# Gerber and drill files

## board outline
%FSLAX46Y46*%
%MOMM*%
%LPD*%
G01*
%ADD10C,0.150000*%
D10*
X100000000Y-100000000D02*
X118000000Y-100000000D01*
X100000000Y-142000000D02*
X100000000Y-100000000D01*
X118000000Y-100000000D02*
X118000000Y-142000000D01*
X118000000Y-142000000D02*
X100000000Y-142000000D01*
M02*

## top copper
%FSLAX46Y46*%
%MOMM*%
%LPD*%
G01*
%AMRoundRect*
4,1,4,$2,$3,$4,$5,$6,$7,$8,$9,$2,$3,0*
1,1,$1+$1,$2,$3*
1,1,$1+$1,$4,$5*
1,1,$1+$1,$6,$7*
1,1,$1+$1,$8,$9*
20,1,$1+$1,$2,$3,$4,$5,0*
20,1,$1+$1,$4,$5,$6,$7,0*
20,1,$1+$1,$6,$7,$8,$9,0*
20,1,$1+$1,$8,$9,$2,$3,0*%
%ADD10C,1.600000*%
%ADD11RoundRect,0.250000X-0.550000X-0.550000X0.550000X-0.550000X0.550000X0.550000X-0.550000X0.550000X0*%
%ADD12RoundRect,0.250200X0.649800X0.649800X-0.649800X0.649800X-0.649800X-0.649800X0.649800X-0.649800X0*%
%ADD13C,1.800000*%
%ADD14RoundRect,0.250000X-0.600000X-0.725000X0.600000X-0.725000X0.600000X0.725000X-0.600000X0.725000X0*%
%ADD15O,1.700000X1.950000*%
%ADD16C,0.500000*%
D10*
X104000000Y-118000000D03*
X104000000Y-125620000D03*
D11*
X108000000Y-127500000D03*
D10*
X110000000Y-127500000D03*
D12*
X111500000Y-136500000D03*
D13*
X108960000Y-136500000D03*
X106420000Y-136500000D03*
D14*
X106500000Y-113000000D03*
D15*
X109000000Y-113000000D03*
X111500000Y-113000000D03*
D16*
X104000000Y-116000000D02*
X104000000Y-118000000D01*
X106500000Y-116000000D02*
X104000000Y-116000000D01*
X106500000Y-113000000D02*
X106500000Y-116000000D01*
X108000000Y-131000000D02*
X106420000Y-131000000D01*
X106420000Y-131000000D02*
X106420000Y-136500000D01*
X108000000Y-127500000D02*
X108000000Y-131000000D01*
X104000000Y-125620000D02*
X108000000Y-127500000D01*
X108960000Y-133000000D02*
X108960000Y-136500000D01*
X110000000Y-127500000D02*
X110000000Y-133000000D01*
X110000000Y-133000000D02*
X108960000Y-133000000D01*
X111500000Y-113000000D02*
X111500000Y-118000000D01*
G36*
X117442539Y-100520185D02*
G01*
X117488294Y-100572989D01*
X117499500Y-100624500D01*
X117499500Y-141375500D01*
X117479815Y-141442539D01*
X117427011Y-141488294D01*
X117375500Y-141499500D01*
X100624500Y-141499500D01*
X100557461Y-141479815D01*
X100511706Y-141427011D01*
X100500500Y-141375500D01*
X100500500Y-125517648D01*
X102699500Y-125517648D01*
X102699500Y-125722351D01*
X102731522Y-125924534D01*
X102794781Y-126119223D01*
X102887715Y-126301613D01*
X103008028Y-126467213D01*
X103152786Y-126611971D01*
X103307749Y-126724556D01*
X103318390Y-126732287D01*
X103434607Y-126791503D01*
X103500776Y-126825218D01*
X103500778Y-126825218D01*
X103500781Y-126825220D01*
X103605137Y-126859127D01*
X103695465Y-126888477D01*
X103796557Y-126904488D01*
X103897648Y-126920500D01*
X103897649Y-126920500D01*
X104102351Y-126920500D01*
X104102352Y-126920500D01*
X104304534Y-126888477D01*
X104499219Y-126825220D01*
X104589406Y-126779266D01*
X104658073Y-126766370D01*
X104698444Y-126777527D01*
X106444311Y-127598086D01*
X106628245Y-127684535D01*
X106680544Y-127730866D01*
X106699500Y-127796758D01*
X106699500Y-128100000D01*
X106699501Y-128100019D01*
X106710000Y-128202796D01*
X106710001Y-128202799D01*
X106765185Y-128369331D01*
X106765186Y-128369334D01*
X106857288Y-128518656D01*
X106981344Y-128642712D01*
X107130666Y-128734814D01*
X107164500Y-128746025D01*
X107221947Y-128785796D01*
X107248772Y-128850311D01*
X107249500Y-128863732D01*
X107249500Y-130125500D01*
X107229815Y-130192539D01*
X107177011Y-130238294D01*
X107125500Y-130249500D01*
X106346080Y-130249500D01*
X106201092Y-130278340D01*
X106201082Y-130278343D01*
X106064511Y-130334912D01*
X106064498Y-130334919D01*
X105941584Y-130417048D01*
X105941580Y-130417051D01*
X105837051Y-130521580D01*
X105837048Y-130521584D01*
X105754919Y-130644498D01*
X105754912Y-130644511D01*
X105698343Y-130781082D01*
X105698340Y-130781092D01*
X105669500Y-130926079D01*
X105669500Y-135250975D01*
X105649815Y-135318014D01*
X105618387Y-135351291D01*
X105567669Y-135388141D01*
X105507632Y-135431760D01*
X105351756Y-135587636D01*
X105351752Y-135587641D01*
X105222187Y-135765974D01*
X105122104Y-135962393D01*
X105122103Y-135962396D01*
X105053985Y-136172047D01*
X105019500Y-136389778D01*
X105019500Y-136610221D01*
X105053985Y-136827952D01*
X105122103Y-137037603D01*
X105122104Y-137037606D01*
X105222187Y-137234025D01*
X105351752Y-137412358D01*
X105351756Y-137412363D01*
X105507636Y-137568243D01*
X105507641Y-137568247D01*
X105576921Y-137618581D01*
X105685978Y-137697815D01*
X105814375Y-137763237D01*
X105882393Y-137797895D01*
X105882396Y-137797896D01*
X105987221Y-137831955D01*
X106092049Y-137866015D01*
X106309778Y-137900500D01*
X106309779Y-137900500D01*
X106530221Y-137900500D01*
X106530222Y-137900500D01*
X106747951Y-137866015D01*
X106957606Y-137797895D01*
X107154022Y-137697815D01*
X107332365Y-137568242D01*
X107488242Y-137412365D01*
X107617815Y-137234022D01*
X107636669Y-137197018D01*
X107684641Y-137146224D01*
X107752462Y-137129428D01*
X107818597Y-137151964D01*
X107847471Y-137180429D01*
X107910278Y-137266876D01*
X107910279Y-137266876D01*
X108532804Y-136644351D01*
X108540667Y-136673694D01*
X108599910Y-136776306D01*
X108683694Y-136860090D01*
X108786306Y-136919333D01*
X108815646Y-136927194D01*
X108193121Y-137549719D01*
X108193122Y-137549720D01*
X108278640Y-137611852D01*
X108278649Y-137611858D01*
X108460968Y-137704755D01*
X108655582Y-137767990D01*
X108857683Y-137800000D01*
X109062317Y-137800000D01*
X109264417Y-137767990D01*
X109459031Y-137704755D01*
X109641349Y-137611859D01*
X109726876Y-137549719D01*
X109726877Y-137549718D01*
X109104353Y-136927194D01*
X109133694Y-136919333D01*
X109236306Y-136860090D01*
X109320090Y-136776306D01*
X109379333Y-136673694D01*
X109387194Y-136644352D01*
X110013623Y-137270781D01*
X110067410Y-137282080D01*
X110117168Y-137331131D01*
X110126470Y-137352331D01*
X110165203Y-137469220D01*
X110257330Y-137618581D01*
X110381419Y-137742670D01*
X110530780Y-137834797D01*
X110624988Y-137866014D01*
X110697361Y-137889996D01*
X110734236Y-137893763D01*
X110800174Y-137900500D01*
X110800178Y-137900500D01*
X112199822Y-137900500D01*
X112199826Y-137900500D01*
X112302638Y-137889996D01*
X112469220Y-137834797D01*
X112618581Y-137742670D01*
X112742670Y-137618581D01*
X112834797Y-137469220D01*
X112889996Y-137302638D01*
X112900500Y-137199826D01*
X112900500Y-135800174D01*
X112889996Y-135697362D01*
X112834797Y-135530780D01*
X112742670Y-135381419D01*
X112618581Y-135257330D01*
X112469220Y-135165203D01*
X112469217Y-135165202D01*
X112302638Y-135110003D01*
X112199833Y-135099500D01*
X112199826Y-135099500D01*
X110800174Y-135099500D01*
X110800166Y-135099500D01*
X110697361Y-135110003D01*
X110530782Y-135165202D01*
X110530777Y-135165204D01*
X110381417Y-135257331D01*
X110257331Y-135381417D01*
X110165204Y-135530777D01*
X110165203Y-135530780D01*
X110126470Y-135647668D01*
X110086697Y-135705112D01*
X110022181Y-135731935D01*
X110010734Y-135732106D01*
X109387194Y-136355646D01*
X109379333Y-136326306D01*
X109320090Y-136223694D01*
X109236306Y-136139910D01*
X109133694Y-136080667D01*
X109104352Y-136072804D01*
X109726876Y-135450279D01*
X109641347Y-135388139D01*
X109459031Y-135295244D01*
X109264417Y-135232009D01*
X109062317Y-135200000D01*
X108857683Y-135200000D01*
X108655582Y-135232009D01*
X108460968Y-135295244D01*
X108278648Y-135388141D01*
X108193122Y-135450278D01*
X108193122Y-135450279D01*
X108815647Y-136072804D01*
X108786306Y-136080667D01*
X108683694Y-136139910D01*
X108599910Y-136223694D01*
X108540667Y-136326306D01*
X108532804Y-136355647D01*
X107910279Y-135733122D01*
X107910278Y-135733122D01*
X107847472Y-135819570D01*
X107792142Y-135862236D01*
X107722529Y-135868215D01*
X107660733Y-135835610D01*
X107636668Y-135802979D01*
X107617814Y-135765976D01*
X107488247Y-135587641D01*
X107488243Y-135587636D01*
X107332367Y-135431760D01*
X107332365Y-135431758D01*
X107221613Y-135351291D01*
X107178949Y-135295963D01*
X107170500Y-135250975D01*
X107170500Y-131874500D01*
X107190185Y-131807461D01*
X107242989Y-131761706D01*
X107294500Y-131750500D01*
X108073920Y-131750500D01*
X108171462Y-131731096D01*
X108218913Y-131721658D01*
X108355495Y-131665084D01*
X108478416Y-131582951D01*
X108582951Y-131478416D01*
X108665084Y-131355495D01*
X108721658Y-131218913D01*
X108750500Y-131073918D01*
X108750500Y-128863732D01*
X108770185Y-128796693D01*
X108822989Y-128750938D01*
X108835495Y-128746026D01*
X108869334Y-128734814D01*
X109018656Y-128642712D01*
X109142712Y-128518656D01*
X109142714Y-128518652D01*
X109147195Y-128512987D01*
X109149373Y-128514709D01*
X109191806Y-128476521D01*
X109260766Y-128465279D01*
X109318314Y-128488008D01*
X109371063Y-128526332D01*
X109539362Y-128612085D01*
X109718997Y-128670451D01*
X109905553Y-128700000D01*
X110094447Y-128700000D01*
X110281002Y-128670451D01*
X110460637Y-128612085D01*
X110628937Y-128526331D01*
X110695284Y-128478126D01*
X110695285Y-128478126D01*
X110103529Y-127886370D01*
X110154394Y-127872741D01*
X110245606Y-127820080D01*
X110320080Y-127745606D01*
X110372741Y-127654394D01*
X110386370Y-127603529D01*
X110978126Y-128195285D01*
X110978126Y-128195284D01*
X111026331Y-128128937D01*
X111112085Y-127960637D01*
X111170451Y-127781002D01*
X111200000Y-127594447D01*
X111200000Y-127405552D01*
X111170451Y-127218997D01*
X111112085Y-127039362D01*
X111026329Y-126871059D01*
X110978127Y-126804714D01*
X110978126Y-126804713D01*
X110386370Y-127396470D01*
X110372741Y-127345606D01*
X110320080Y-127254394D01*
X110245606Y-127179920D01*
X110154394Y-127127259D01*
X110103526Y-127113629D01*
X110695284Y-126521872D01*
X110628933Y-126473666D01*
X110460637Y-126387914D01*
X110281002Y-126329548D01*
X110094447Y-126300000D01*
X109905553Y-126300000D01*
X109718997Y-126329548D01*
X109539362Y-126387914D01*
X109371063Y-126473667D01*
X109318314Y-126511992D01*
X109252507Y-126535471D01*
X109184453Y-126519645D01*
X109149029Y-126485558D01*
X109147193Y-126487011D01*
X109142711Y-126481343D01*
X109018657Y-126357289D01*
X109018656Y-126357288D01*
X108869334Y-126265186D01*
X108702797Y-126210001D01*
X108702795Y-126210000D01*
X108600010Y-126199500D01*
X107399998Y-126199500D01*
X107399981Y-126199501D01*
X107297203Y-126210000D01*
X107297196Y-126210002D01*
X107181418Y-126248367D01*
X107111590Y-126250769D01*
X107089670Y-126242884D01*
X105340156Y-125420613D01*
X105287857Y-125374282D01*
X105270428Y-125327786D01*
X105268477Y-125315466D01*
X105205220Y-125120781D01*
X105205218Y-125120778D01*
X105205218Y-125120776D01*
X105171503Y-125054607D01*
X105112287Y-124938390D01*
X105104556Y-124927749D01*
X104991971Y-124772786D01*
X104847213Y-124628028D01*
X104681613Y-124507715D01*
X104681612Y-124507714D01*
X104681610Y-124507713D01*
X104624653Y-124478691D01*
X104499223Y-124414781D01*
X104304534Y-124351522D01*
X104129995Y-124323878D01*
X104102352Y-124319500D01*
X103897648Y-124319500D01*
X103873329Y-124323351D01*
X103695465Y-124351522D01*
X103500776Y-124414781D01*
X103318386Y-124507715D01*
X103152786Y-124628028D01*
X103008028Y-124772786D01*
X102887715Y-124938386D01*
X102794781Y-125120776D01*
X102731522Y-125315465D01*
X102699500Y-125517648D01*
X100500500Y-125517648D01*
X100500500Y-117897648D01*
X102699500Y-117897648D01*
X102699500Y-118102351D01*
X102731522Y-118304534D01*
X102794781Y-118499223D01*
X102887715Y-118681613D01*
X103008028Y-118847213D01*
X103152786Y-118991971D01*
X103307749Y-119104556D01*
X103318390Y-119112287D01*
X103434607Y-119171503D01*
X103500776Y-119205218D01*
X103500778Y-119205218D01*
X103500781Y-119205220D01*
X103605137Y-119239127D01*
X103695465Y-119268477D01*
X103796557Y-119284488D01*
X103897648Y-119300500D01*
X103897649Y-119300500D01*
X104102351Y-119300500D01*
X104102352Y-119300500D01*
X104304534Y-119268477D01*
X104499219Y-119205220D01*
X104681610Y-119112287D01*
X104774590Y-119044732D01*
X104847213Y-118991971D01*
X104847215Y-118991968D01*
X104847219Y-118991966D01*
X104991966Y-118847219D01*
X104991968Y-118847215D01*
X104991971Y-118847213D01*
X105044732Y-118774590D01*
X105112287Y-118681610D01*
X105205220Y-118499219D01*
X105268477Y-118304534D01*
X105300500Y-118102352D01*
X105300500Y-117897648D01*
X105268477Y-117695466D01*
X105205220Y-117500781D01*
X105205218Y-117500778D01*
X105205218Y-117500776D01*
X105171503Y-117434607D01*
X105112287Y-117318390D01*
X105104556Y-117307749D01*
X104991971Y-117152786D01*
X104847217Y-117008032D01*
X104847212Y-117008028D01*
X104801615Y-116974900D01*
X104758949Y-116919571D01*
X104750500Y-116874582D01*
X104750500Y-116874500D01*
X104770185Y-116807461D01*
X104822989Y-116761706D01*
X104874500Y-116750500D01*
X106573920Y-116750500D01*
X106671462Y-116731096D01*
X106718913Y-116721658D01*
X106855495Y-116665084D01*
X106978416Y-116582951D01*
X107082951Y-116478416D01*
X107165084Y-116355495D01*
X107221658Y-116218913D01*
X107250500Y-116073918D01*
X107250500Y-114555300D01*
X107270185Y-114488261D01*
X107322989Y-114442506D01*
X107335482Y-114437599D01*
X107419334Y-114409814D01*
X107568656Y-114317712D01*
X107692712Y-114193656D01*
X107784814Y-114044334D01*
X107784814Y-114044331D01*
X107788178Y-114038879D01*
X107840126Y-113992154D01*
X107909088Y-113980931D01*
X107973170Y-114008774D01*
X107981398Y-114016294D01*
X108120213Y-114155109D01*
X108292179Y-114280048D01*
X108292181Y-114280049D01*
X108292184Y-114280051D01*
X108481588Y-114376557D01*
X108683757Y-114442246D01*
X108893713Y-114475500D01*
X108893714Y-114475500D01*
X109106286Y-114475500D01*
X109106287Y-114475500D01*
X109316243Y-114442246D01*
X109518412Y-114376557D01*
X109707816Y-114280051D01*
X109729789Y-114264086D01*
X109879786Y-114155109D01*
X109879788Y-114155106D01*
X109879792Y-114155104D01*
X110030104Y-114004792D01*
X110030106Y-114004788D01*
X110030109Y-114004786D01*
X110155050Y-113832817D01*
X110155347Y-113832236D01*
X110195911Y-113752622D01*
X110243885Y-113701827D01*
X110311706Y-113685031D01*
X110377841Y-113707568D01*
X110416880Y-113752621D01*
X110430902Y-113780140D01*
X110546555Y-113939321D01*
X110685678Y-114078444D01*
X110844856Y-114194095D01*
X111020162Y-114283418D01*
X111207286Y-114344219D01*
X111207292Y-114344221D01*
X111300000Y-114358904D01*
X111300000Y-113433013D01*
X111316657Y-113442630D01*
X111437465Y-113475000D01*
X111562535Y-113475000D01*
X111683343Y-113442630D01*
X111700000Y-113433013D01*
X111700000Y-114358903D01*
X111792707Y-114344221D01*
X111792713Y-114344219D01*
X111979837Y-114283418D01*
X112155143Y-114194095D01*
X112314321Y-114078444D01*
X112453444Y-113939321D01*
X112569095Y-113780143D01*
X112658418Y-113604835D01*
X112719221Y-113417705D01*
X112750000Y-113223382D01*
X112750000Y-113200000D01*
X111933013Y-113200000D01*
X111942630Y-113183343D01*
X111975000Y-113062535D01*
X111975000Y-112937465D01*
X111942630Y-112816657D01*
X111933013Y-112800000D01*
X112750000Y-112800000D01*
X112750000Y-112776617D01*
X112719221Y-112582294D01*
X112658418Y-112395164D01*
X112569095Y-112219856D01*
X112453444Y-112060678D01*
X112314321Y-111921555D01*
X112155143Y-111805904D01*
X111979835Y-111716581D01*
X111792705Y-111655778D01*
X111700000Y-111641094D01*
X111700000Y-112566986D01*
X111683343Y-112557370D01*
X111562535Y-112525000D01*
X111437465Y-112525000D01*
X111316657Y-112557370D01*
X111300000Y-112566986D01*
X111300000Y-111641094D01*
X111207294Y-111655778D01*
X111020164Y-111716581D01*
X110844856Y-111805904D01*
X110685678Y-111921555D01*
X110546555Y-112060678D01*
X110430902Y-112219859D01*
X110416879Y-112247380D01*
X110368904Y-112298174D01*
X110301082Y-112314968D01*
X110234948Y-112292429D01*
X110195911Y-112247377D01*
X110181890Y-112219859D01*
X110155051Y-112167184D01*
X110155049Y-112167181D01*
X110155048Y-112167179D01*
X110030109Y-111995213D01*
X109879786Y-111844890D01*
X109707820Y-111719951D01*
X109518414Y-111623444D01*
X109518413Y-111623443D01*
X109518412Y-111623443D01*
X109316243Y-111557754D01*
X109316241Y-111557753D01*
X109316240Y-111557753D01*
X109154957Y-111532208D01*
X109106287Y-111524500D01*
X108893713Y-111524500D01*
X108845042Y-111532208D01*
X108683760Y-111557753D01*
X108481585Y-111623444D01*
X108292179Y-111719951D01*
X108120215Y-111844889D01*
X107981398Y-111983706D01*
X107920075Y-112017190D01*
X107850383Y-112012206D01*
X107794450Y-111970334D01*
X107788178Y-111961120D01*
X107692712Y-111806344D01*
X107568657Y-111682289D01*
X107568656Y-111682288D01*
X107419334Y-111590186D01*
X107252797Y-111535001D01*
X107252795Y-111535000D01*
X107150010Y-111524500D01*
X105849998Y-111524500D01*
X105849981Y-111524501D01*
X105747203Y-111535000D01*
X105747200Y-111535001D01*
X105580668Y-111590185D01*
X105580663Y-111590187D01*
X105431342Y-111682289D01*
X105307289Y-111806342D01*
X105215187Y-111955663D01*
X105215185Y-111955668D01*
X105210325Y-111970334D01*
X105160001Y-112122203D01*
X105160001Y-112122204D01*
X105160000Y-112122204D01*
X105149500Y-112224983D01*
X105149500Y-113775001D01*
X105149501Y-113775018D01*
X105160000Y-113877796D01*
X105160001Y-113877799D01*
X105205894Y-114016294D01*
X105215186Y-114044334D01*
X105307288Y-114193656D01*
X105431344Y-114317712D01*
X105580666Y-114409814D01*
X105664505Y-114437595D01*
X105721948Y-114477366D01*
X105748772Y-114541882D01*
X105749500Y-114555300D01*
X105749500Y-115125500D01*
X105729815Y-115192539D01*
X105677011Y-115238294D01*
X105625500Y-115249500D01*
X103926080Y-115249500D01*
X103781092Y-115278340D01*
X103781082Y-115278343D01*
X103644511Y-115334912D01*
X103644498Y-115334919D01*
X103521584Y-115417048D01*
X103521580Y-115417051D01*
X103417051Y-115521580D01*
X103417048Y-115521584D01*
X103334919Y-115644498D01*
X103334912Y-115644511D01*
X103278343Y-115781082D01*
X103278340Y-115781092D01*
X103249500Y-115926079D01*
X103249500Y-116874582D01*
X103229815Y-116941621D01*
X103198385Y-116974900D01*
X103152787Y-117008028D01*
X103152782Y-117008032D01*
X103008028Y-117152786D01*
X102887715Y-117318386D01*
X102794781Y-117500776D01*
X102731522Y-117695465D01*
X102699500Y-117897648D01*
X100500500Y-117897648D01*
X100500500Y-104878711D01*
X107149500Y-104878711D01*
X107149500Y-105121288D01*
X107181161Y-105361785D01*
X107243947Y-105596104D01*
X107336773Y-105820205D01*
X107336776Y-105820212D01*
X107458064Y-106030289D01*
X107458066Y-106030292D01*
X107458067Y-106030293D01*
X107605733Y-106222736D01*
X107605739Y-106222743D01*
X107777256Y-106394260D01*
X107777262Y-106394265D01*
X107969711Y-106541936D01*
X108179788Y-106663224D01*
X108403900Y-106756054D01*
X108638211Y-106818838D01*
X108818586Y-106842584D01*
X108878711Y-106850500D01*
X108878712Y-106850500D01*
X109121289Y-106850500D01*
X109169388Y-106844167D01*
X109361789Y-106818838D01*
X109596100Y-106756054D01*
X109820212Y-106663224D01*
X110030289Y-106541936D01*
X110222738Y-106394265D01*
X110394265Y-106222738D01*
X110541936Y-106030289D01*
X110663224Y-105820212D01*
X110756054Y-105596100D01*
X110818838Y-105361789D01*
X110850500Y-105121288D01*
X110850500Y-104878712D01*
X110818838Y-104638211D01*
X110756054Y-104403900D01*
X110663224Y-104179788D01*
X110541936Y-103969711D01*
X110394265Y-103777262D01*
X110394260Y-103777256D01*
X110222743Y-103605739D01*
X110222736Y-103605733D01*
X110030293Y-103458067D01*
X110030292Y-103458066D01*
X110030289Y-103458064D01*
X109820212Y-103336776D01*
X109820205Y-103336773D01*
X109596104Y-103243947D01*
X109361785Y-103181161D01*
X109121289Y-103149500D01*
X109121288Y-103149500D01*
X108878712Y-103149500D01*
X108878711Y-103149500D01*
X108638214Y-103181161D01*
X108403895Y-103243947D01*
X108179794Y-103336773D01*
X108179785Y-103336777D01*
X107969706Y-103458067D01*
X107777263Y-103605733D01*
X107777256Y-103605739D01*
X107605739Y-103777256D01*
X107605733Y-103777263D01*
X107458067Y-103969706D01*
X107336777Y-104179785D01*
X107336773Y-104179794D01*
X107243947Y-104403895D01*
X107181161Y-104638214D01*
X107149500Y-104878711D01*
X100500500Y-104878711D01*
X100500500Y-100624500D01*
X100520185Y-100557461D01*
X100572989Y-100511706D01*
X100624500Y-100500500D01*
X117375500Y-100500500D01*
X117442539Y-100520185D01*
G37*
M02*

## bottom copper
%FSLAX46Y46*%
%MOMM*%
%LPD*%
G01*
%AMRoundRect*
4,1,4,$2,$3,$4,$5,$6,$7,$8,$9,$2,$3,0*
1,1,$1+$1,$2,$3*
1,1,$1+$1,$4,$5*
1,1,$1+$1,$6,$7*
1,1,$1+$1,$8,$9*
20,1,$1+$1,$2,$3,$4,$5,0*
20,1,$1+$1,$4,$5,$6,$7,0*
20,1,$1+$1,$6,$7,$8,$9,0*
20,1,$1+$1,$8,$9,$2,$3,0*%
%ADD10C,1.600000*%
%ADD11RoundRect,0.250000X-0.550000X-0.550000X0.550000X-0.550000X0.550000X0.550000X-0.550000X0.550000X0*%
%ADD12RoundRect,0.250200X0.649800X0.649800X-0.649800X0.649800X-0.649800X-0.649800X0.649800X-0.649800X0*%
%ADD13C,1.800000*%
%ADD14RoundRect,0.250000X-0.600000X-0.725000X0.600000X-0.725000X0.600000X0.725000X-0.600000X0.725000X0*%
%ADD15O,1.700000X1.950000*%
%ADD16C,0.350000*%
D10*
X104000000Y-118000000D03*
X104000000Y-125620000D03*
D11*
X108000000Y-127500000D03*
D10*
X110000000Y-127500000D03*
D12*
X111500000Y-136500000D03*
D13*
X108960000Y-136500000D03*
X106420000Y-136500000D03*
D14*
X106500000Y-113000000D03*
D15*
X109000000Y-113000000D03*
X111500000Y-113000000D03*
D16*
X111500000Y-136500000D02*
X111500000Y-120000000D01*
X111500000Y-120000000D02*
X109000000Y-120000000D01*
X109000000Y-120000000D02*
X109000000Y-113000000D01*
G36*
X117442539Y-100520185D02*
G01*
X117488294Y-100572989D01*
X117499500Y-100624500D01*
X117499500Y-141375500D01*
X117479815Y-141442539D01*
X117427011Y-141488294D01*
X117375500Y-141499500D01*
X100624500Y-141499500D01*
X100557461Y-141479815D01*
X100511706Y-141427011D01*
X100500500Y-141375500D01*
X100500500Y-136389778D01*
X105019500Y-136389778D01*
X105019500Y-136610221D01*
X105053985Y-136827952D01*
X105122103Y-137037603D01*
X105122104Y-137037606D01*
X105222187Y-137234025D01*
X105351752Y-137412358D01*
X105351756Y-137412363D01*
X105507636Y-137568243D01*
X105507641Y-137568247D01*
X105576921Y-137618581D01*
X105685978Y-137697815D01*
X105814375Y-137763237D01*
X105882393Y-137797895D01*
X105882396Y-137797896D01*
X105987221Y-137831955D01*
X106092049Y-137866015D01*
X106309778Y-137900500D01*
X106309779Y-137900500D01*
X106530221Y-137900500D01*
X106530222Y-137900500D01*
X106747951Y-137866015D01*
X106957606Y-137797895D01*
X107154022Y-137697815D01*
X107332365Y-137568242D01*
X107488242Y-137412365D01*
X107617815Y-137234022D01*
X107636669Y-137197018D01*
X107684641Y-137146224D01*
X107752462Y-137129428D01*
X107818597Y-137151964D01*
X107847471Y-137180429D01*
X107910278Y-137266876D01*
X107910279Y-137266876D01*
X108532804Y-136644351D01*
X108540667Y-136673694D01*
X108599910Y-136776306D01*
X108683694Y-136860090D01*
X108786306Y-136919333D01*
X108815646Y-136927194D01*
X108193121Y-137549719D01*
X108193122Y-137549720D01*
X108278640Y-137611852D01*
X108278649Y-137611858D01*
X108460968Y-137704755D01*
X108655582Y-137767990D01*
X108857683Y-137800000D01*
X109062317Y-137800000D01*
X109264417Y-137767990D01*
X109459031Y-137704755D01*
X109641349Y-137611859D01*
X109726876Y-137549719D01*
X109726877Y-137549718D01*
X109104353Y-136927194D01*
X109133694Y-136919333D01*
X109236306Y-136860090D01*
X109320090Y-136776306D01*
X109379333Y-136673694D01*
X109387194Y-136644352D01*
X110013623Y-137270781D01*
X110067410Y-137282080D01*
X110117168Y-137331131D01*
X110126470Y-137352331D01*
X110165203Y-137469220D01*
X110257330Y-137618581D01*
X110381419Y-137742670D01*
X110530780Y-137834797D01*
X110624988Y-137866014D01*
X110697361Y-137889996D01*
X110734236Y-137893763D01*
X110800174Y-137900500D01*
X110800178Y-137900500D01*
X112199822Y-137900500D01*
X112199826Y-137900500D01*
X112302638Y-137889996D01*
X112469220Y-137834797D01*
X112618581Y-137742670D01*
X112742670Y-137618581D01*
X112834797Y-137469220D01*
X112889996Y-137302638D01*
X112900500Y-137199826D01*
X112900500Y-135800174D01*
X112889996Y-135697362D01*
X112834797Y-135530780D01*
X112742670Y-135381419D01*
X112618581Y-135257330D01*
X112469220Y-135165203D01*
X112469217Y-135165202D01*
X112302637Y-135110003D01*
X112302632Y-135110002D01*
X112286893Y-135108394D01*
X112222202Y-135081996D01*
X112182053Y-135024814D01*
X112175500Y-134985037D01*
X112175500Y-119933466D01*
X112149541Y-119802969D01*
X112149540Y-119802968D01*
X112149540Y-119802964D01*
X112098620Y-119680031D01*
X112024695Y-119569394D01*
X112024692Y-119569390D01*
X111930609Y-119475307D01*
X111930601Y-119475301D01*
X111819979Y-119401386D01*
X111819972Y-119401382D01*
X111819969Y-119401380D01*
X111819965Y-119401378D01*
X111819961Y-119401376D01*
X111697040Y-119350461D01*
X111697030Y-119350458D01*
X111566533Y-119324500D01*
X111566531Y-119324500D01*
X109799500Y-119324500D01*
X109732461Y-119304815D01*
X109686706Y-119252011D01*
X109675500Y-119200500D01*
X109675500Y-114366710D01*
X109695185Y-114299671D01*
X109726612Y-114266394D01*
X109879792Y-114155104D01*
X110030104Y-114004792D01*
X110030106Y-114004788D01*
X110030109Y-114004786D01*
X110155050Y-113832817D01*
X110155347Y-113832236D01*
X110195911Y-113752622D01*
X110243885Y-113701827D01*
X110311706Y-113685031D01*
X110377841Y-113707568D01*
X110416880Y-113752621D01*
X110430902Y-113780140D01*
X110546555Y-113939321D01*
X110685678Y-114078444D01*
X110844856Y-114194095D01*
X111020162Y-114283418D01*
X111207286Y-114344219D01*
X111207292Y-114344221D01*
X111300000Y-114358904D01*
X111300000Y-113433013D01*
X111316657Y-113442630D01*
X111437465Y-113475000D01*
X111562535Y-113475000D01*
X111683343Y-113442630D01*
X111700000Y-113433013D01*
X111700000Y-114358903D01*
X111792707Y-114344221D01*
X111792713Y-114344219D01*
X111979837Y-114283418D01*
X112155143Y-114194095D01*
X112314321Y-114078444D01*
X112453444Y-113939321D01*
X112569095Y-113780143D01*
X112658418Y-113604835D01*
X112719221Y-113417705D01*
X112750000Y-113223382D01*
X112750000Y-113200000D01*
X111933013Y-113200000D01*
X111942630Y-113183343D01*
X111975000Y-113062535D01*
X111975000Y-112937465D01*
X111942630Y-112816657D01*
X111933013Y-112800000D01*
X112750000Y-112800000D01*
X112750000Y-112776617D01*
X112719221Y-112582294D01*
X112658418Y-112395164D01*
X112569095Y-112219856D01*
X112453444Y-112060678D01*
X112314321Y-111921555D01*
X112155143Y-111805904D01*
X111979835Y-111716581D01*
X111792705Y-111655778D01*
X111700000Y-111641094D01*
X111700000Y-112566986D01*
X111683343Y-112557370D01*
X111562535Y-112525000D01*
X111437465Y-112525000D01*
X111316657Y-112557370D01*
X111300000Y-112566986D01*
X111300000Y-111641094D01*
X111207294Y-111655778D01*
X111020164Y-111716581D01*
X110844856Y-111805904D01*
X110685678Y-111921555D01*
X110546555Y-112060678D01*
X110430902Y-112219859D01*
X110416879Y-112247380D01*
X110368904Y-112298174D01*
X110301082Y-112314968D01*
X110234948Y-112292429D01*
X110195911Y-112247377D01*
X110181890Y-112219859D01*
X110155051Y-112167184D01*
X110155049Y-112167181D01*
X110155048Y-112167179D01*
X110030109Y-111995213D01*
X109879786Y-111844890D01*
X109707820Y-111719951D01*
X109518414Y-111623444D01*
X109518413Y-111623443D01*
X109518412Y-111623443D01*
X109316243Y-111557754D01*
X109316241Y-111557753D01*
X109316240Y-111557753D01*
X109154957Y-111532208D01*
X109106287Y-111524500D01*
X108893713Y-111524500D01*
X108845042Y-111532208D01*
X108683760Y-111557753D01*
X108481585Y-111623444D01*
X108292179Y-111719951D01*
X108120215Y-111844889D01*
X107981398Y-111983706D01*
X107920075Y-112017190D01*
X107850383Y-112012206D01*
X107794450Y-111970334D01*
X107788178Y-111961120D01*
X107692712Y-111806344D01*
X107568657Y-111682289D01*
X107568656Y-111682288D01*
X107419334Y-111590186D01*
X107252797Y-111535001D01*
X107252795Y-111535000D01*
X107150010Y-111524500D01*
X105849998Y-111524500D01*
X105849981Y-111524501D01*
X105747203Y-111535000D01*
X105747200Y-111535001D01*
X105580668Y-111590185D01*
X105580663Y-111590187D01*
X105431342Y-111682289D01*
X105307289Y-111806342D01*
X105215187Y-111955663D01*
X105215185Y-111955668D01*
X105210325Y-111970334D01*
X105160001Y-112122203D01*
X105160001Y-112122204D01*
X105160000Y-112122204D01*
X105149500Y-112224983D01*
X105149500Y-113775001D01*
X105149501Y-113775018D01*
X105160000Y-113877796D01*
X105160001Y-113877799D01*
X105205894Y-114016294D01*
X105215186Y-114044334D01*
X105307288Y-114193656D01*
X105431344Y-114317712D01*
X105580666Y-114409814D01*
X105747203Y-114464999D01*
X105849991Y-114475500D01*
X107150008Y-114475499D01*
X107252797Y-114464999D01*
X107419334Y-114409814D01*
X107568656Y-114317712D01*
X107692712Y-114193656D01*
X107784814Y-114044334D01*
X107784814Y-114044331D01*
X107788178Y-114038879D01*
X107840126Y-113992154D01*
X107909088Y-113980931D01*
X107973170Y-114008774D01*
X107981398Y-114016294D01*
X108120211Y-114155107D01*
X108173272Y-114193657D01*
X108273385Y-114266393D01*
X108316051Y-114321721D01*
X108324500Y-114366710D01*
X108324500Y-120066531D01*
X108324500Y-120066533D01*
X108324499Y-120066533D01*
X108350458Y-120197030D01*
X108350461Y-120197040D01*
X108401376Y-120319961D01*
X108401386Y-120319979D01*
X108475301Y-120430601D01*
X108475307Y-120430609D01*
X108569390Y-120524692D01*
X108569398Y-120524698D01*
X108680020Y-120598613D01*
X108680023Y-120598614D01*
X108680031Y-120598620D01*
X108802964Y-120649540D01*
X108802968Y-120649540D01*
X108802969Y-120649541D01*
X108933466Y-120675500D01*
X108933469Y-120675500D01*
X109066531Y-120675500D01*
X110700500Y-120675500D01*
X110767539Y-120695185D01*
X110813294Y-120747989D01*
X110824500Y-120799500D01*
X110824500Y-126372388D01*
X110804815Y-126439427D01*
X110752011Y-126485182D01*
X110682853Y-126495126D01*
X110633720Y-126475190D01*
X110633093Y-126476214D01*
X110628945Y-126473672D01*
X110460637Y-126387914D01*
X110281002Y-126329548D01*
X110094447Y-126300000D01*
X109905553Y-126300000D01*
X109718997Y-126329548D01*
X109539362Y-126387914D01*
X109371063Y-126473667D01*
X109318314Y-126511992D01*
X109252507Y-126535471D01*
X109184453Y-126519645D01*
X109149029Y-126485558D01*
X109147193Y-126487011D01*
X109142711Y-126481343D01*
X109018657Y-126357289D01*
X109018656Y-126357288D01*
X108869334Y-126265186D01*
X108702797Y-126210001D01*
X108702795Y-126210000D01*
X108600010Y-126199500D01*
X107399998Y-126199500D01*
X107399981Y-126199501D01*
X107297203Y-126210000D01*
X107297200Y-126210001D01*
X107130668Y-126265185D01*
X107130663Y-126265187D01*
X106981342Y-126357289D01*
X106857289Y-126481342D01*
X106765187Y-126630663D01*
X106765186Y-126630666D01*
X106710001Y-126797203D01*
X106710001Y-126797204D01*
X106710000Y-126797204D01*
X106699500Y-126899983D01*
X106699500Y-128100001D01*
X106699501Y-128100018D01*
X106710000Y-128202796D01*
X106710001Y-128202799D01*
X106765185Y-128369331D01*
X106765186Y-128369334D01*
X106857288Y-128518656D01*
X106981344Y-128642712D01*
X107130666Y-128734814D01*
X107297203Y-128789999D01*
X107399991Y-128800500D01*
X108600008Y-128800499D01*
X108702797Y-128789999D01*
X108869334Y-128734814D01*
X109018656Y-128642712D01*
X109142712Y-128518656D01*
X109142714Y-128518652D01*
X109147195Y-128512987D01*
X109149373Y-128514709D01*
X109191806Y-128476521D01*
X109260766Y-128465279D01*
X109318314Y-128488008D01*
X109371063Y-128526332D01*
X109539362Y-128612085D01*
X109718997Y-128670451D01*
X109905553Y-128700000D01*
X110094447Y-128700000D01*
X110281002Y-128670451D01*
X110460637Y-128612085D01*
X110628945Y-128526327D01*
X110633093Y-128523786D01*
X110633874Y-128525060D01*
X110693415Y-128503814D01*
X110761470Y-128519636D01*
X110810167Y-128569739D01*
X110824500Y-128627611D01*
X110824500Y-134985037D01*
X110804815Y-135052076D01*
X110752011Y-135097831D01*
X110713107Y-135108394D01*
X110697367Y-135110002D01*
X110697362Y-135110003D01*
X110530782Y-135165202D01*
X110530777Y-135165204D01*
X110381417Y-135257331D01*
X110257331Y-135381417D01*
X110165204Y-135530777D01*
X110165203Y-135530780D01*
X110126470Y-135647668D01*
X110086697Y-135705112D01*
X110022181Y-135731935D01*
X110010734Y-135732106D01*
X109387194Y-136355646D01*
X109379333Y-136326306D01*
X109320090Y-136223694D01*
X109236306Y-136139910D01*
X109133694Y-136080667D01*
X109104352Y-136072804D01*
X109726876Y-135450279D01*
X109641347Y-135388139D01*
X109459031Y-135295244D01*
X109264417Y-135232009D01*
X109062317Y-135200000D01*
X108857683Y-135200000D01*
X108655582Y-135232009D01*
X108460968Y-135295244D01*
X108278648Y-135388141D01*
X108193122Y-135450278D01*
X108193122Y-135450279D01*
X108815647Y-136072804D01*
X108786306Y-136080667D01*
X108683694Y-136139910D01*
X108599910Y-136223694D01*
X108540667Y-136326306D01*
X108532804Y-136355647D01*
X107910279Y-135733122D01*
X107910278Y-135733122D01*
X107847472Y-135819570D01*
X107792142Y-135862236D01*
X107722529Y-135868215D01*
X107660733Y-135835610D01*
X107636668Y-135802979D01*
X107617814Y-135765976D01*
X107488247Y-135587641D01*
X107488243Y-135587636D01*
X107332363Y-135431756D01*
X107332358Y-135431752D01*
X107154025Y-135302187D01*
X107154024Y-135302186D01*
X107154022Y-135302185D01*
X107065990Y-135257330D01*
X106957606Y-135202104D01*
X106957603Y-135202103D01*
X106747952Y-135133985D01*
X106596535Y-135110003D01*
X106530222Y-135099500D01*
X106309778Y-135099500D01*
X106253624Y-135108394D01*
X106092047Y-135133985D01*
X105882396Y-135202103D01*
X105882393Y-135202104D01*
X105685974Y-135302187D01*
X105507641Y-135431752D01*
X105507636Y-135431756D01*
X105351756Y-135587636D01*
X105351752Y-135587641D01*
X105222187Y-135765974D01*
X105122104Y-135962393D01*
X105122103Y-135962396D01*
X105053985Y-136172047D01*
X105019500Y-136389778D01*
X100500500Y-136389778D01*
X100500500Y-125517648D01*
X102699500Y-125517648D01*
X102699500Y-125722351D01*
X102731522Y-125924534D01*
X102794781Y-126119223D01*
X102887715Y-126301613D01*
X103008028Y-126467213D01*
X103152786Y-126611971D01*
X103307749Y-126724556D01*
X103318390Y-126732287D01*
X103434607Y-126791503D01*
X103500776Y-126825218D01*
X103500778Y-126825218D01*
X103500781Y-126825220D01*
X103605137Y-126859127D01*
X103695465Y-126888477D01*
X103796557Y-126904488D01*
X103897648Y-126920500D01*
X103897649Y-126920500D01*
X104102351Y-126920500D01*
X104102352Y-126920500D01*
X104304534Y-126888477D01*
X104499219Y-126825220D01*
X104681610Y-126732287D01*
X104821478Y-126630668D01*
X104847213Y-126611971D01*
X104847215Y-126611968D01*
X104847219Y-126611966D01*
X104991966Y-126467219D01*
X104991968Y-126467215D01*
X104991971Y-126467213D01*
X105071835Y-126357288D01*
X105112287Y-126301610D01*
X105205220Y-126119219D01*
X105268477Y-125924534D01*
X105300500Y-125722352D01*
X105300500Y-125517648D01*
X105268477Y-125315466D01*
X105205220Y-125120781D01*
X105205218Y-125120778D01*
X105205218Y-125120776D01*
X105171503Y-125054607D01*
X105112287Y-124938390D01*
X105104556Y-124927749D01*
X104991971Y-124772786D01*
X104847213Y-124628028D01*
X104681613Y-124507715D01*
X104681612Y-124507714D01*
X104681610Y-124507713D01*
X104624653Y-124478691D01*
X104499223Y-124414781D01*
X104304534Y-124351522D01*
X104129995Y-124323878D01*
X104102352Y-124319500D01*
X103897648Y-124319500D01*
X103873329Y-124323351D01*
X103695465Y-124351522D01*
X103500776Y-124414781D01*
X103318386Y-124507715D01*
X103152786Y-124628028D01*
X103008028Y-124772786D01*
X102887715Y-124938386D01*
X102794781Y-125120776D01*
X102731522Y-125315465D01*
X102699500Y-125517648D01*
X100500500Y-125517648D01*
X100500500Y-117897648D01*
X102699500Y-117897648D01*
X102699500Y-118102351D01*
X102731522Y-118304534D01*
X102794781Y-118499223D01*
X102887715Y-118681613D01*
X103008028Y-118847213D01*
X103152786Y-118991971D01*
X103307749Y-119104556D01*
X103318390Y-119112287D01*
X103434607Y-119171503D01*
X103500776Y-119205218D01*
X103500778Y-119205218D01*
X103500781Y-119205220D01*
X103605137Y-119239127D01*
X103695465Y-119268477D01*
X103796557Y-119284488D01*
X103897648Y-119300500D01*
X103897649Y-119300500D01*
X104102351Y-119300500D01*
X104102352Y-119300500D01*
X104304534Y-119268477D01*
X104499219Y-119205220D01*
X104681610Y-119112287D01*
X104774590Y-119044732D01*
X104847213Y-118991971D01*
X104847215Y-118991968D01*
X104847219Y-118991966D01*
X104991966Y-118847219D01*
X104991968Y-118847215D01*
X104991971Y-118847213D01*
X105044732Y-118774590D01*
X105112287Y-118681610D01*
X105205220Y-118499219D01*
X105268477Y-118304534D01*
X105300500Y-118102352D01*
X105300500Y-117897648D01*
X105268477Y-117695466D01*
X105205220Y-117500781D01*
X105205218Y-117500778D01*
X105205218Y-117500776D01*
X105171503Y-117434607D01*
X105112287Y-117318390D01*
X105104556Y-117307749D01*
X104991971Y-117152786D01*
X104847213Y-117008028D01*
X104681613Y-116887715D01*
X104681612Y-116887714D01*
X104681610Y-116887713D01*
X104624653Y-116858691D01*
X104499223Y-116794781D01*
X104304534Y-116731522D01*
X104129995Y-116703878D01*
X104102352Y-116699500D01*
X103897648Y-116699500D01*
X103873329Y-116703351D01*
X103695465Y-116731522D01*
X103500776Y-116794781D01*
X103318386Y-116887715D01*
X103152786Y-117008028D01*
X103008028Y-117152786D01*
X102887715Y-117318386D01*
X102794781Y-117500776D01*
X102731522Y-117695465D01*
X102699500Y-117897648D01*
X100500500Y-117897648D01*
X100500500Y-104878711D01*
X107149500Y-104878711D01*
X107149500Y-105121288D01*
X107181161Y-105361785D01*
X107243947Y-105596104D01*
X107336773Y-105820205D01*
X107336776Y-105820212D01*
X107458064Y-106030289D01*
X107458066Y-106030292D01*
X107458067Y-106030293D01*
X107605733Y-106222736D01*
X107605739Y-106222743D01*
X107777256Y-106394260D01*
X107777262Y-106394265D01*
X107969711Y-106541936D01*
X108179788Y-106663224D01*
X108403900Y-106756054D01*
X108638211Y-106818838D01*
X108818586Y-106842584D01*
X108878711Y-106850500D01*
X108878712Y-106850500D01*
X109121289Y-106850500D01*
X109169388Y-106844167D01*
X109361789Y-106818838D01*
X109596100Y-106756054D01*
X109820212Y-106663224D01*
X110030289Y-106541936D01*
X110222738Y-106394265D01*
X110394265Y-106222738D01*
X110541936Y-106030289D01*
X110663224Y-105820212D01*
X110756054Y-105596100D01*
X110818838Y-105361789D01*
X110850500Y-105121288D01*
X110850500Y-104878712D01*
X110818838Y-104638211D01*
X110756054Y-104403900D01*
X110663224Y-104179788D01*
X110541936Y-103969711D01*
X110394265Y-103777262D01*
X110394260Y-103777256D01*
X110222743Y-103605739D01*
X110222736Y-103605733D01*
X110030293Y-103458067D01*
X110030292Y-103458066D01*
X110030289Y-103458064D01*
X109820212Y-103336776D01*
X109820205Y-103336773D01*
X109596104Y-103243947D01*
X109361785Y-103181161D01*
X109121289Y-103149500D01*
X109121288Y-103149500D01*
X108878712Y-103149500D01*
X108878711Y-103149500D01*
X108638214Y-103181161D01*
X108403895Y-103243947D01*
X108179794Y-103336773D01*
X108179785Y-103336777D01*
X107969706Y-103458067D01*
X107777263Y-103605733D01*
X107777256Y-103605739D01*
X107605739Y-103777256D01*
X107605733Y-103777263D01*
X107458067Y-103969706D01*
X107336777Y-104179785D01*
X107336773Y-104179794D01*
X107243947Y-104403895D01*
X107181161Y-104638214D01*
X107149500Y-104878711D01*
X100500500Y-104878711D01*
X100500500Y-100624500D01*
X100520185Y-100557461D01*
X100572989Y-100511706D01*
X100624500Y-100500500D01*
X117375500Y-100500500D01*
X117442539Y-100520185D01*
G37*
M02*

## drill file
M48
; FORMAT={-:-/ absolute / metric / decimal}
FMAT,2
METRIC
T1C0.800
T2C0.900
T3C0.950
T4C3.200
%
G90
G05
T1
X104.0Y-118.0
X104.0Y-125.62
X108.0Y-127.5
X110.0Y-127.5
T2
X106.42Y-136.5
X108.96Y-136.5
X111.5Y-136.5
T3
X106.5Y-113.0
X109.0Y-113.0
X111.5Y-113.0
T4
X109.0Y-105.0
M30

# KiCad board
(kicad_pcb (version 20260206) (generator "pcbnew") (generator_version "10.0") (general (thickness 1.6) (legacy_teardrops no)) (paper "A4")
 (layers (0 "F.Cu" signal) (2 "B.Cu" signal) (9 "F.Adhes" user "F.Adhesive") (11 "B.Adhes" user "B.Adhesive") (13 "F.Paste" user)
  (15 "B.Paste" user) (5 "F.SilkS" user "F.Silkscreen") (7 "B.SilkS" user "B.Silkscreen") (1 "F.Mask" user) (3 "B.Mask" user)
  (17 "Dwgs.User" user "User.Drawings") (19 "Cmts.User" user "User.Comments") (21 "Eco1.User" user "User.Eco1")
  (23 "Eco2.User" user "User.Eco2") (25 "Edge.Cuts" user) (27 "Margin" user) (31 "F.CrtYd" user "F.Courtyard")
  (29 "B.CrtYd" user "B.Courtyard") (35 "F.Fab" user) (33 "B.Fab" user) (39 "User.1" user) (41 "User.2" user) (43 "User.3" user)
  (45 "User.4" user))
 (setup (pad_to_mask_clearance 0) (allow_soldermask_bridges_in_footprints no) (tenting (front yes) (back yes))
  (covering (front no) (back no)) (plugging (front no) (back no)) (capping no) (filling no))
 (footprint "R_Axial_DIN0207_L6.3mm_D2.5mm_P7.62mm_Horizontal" (layer "F.Cu") (at 104 118 -90)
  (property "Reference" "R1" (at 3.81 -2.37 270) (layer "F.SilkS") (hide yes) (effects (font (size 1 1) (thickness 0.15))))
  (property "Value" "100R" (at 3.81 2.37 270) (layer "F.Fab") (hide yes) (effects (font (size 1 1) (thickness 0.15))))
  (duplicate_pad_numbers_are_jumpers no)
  (pad "1" thru_hole circle (at 0 0 270) (size 1.6 1.6) (drill 0.8) (layers "*.Cu" "*.Mask") (remove_unused_layers no) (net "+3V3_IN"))
  (pad "2" thru_hole circle (at 7.62 0 270) (size 1.6 1.6) (drill 0.8) (layers "*.Cu" "*.Mask") (remove_unused_layers no) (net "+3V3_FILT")))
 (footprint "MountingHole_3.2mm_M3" (layer "F.Cu") (at 109 105)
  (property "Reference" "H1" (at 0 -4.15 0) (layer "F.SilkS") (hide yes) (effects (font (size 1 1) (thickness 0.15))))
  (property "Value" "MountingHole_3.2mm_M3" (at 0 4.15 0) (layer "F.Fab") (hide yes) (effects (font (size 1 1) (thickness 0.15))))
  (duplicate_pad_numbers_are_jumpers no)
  (pad "" np_thru_hole circle (at 0 0) (size 3.2 3.2) (drill 3.2) (layers "*.Cu" "*.Mask")))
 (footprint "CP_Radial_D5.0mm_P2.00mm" (layer "F.Cu") (at 108 127.5)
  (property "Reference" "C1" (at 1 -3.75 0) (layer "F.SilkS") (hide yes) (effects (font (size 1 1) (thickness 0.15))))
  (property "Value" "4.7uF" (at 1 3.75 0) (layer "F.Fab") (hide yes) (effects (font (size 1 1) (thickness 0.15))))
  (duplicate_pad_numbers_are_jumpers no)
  (pad "1" thru_hole roundrect (at 0 0) (size 1.6 1.6) (drill 0.8) (layers "*.Cu" "*.Mask") (remove_unused_layers no)
   (roundrect_rratio 0.15625) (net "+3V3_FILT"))
  (pad "2" thru_hole circle (at 2 0) (size 1.6 1.6) (drill 0.8) (layers "*.Cu" "*.Mask") (remove_unused_layers no) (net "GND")))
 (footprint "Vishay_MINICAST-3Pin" (layer "F.Cu") (at 111.5 136.5 180)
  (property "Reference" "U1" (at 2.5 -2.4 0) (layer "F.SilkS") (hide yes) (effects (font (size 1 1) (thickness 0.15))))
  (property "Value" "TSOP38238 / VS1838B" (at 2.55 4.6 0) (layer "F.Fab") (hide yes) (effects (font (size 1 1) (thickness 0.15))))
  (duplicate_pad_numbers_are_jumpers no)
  (pad "1" thru_hole roundrect (at 0 0 180) (size 1.8 1.8) (drill 0.9) (layers "*.Cu" "*.Mask") (remove_unused_layers no)
   (roundrect_rratio 0.139) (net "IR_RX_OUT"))
  (pad "2" thru_hole circle (at 2.54 0 180) (size 1.8 1.8) (drill 0.9) (layers "*.Cu" "*.Mask") (remove_unused_layers no) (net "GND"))
  (pad "3" thru_hole circle (at 5.08 0 180) (size 1.8 1.8) (drill 0.9) (layers "*.Cu" "*.Mask") (remove_unused_layers no) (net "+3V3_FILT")))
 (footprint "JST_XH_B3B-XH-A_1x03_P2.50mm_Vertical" (layer "F.Cu") (at 106.5 113)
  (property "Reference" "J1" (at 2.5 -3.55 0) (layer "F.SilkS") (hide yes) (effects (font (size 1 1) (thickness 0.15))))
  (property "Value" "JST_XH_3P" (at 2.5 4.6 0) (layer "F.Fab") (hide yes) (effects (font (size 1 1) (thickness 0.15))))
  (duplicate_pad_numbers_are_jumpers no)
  (pad "1" thru_hole roundrect (at 0 0) (size 1.7 1.95) (drill 0.95) (layers "*.Cu" "*.Mask") (remove_unused_layers no)
   (roundrect_rratio 0.147059) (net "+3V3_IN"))
  (pad "2" thru_hole oval (at 2.5 0) (size 1.7 1.95) (drill 0.95) (layers "*.Cu" "*.Mask") (remove_unused_layers no) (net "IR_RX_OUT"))
  (pad "3" thru_hole oval (at 5 0) (size 1.7 1.95) (drill 0.95) (layers "*.Cu" "*.Mask") (remove_unused_layers no) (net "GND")))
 (gr_line (start 100 100) (end 118 100) (stroke (width 0.15) (type default)) (layer "Edge.Cuts"))
 (gr_line (start 100 142) (end 100 100) (stroke (width 0.15) (type default)) (layer "Edge.Cuts"))
 (gr_line (start 118 100) (end 118 142) (stroke (width 0.15) (type default)) (layer "Edge.Cuts"))
 (gr_line (start 118 142) (end 100 142) (stroke (width 0.15) (type default)) (layer "Edge.Cuts"))
 (segment (start 104 116) (end 104 118) (width 0.5) (layer "F.Cu") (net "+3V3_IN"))
 (segment (start 106.5 116) (end 104 116) (width 0.5) (layer "F.Cu") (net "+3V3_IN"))
 (segment (start 106.5 113) (end 106.5 116) (width 0.5) (layer "F.Cu") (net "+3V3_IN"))
 (segment (start 108 131) (end 106.42 131) (width 0.5) (layer "F.Cu") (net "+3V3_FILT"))
 (segment (start 106.42 131) (end 106.42 136.5) (width 0.5) (layer "F.Cu") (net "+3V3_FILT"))
 (segment (start 108 127.5) (end 108 131) (width 0.5) (layer "F.Cu") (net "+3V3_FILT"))
 (segment (start 104 125.62) (end 108 127.5) (width 0.5) (layer "F.Cu") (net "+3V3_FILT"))
 (segment (start 111.5 136.5) (end 111.5 120) (width 0.35) (layer "B.Cu") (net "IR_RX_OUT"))
 (segment (start 111.5 120) (end 109 120) (width 0.35) (layer "B.Cu") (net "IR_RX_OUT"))
 (segment (start 109 120) (end 109 113) (width 0.35) (layer "B.Cu") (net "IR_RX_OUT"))
 (segment (start 108.96 133) (end 108.96 136.5) (width 0.5) (layer "F.Cu") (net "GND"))
 (segment (start 110 127.5) (end 110 133) (width 0.5) (layer "F.Cu") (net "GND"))
 (segment (start 110 133) (end 108.96 133) (width 0.5) (layer "F.Cu") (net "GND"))
 (segment (start 111.5 113) (end 111.5 118) (width 0.5) (layer "F.Cu") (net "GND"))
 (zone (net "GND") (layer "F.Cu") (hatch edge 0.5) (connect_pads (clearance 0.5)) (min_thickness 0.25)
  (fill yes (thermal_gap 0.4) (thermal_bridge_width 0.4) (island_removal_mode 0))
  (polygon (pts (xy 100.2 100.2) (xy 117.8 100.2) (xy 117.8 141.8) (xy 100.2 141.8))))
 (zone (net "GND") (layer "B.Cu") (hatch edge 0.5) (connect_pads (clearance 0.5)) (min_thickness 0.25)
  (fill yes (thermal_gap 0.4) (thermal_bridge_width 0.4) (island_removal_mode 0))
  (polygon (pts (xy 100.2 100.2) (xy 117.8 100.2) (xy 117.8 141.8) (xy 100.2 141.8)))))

